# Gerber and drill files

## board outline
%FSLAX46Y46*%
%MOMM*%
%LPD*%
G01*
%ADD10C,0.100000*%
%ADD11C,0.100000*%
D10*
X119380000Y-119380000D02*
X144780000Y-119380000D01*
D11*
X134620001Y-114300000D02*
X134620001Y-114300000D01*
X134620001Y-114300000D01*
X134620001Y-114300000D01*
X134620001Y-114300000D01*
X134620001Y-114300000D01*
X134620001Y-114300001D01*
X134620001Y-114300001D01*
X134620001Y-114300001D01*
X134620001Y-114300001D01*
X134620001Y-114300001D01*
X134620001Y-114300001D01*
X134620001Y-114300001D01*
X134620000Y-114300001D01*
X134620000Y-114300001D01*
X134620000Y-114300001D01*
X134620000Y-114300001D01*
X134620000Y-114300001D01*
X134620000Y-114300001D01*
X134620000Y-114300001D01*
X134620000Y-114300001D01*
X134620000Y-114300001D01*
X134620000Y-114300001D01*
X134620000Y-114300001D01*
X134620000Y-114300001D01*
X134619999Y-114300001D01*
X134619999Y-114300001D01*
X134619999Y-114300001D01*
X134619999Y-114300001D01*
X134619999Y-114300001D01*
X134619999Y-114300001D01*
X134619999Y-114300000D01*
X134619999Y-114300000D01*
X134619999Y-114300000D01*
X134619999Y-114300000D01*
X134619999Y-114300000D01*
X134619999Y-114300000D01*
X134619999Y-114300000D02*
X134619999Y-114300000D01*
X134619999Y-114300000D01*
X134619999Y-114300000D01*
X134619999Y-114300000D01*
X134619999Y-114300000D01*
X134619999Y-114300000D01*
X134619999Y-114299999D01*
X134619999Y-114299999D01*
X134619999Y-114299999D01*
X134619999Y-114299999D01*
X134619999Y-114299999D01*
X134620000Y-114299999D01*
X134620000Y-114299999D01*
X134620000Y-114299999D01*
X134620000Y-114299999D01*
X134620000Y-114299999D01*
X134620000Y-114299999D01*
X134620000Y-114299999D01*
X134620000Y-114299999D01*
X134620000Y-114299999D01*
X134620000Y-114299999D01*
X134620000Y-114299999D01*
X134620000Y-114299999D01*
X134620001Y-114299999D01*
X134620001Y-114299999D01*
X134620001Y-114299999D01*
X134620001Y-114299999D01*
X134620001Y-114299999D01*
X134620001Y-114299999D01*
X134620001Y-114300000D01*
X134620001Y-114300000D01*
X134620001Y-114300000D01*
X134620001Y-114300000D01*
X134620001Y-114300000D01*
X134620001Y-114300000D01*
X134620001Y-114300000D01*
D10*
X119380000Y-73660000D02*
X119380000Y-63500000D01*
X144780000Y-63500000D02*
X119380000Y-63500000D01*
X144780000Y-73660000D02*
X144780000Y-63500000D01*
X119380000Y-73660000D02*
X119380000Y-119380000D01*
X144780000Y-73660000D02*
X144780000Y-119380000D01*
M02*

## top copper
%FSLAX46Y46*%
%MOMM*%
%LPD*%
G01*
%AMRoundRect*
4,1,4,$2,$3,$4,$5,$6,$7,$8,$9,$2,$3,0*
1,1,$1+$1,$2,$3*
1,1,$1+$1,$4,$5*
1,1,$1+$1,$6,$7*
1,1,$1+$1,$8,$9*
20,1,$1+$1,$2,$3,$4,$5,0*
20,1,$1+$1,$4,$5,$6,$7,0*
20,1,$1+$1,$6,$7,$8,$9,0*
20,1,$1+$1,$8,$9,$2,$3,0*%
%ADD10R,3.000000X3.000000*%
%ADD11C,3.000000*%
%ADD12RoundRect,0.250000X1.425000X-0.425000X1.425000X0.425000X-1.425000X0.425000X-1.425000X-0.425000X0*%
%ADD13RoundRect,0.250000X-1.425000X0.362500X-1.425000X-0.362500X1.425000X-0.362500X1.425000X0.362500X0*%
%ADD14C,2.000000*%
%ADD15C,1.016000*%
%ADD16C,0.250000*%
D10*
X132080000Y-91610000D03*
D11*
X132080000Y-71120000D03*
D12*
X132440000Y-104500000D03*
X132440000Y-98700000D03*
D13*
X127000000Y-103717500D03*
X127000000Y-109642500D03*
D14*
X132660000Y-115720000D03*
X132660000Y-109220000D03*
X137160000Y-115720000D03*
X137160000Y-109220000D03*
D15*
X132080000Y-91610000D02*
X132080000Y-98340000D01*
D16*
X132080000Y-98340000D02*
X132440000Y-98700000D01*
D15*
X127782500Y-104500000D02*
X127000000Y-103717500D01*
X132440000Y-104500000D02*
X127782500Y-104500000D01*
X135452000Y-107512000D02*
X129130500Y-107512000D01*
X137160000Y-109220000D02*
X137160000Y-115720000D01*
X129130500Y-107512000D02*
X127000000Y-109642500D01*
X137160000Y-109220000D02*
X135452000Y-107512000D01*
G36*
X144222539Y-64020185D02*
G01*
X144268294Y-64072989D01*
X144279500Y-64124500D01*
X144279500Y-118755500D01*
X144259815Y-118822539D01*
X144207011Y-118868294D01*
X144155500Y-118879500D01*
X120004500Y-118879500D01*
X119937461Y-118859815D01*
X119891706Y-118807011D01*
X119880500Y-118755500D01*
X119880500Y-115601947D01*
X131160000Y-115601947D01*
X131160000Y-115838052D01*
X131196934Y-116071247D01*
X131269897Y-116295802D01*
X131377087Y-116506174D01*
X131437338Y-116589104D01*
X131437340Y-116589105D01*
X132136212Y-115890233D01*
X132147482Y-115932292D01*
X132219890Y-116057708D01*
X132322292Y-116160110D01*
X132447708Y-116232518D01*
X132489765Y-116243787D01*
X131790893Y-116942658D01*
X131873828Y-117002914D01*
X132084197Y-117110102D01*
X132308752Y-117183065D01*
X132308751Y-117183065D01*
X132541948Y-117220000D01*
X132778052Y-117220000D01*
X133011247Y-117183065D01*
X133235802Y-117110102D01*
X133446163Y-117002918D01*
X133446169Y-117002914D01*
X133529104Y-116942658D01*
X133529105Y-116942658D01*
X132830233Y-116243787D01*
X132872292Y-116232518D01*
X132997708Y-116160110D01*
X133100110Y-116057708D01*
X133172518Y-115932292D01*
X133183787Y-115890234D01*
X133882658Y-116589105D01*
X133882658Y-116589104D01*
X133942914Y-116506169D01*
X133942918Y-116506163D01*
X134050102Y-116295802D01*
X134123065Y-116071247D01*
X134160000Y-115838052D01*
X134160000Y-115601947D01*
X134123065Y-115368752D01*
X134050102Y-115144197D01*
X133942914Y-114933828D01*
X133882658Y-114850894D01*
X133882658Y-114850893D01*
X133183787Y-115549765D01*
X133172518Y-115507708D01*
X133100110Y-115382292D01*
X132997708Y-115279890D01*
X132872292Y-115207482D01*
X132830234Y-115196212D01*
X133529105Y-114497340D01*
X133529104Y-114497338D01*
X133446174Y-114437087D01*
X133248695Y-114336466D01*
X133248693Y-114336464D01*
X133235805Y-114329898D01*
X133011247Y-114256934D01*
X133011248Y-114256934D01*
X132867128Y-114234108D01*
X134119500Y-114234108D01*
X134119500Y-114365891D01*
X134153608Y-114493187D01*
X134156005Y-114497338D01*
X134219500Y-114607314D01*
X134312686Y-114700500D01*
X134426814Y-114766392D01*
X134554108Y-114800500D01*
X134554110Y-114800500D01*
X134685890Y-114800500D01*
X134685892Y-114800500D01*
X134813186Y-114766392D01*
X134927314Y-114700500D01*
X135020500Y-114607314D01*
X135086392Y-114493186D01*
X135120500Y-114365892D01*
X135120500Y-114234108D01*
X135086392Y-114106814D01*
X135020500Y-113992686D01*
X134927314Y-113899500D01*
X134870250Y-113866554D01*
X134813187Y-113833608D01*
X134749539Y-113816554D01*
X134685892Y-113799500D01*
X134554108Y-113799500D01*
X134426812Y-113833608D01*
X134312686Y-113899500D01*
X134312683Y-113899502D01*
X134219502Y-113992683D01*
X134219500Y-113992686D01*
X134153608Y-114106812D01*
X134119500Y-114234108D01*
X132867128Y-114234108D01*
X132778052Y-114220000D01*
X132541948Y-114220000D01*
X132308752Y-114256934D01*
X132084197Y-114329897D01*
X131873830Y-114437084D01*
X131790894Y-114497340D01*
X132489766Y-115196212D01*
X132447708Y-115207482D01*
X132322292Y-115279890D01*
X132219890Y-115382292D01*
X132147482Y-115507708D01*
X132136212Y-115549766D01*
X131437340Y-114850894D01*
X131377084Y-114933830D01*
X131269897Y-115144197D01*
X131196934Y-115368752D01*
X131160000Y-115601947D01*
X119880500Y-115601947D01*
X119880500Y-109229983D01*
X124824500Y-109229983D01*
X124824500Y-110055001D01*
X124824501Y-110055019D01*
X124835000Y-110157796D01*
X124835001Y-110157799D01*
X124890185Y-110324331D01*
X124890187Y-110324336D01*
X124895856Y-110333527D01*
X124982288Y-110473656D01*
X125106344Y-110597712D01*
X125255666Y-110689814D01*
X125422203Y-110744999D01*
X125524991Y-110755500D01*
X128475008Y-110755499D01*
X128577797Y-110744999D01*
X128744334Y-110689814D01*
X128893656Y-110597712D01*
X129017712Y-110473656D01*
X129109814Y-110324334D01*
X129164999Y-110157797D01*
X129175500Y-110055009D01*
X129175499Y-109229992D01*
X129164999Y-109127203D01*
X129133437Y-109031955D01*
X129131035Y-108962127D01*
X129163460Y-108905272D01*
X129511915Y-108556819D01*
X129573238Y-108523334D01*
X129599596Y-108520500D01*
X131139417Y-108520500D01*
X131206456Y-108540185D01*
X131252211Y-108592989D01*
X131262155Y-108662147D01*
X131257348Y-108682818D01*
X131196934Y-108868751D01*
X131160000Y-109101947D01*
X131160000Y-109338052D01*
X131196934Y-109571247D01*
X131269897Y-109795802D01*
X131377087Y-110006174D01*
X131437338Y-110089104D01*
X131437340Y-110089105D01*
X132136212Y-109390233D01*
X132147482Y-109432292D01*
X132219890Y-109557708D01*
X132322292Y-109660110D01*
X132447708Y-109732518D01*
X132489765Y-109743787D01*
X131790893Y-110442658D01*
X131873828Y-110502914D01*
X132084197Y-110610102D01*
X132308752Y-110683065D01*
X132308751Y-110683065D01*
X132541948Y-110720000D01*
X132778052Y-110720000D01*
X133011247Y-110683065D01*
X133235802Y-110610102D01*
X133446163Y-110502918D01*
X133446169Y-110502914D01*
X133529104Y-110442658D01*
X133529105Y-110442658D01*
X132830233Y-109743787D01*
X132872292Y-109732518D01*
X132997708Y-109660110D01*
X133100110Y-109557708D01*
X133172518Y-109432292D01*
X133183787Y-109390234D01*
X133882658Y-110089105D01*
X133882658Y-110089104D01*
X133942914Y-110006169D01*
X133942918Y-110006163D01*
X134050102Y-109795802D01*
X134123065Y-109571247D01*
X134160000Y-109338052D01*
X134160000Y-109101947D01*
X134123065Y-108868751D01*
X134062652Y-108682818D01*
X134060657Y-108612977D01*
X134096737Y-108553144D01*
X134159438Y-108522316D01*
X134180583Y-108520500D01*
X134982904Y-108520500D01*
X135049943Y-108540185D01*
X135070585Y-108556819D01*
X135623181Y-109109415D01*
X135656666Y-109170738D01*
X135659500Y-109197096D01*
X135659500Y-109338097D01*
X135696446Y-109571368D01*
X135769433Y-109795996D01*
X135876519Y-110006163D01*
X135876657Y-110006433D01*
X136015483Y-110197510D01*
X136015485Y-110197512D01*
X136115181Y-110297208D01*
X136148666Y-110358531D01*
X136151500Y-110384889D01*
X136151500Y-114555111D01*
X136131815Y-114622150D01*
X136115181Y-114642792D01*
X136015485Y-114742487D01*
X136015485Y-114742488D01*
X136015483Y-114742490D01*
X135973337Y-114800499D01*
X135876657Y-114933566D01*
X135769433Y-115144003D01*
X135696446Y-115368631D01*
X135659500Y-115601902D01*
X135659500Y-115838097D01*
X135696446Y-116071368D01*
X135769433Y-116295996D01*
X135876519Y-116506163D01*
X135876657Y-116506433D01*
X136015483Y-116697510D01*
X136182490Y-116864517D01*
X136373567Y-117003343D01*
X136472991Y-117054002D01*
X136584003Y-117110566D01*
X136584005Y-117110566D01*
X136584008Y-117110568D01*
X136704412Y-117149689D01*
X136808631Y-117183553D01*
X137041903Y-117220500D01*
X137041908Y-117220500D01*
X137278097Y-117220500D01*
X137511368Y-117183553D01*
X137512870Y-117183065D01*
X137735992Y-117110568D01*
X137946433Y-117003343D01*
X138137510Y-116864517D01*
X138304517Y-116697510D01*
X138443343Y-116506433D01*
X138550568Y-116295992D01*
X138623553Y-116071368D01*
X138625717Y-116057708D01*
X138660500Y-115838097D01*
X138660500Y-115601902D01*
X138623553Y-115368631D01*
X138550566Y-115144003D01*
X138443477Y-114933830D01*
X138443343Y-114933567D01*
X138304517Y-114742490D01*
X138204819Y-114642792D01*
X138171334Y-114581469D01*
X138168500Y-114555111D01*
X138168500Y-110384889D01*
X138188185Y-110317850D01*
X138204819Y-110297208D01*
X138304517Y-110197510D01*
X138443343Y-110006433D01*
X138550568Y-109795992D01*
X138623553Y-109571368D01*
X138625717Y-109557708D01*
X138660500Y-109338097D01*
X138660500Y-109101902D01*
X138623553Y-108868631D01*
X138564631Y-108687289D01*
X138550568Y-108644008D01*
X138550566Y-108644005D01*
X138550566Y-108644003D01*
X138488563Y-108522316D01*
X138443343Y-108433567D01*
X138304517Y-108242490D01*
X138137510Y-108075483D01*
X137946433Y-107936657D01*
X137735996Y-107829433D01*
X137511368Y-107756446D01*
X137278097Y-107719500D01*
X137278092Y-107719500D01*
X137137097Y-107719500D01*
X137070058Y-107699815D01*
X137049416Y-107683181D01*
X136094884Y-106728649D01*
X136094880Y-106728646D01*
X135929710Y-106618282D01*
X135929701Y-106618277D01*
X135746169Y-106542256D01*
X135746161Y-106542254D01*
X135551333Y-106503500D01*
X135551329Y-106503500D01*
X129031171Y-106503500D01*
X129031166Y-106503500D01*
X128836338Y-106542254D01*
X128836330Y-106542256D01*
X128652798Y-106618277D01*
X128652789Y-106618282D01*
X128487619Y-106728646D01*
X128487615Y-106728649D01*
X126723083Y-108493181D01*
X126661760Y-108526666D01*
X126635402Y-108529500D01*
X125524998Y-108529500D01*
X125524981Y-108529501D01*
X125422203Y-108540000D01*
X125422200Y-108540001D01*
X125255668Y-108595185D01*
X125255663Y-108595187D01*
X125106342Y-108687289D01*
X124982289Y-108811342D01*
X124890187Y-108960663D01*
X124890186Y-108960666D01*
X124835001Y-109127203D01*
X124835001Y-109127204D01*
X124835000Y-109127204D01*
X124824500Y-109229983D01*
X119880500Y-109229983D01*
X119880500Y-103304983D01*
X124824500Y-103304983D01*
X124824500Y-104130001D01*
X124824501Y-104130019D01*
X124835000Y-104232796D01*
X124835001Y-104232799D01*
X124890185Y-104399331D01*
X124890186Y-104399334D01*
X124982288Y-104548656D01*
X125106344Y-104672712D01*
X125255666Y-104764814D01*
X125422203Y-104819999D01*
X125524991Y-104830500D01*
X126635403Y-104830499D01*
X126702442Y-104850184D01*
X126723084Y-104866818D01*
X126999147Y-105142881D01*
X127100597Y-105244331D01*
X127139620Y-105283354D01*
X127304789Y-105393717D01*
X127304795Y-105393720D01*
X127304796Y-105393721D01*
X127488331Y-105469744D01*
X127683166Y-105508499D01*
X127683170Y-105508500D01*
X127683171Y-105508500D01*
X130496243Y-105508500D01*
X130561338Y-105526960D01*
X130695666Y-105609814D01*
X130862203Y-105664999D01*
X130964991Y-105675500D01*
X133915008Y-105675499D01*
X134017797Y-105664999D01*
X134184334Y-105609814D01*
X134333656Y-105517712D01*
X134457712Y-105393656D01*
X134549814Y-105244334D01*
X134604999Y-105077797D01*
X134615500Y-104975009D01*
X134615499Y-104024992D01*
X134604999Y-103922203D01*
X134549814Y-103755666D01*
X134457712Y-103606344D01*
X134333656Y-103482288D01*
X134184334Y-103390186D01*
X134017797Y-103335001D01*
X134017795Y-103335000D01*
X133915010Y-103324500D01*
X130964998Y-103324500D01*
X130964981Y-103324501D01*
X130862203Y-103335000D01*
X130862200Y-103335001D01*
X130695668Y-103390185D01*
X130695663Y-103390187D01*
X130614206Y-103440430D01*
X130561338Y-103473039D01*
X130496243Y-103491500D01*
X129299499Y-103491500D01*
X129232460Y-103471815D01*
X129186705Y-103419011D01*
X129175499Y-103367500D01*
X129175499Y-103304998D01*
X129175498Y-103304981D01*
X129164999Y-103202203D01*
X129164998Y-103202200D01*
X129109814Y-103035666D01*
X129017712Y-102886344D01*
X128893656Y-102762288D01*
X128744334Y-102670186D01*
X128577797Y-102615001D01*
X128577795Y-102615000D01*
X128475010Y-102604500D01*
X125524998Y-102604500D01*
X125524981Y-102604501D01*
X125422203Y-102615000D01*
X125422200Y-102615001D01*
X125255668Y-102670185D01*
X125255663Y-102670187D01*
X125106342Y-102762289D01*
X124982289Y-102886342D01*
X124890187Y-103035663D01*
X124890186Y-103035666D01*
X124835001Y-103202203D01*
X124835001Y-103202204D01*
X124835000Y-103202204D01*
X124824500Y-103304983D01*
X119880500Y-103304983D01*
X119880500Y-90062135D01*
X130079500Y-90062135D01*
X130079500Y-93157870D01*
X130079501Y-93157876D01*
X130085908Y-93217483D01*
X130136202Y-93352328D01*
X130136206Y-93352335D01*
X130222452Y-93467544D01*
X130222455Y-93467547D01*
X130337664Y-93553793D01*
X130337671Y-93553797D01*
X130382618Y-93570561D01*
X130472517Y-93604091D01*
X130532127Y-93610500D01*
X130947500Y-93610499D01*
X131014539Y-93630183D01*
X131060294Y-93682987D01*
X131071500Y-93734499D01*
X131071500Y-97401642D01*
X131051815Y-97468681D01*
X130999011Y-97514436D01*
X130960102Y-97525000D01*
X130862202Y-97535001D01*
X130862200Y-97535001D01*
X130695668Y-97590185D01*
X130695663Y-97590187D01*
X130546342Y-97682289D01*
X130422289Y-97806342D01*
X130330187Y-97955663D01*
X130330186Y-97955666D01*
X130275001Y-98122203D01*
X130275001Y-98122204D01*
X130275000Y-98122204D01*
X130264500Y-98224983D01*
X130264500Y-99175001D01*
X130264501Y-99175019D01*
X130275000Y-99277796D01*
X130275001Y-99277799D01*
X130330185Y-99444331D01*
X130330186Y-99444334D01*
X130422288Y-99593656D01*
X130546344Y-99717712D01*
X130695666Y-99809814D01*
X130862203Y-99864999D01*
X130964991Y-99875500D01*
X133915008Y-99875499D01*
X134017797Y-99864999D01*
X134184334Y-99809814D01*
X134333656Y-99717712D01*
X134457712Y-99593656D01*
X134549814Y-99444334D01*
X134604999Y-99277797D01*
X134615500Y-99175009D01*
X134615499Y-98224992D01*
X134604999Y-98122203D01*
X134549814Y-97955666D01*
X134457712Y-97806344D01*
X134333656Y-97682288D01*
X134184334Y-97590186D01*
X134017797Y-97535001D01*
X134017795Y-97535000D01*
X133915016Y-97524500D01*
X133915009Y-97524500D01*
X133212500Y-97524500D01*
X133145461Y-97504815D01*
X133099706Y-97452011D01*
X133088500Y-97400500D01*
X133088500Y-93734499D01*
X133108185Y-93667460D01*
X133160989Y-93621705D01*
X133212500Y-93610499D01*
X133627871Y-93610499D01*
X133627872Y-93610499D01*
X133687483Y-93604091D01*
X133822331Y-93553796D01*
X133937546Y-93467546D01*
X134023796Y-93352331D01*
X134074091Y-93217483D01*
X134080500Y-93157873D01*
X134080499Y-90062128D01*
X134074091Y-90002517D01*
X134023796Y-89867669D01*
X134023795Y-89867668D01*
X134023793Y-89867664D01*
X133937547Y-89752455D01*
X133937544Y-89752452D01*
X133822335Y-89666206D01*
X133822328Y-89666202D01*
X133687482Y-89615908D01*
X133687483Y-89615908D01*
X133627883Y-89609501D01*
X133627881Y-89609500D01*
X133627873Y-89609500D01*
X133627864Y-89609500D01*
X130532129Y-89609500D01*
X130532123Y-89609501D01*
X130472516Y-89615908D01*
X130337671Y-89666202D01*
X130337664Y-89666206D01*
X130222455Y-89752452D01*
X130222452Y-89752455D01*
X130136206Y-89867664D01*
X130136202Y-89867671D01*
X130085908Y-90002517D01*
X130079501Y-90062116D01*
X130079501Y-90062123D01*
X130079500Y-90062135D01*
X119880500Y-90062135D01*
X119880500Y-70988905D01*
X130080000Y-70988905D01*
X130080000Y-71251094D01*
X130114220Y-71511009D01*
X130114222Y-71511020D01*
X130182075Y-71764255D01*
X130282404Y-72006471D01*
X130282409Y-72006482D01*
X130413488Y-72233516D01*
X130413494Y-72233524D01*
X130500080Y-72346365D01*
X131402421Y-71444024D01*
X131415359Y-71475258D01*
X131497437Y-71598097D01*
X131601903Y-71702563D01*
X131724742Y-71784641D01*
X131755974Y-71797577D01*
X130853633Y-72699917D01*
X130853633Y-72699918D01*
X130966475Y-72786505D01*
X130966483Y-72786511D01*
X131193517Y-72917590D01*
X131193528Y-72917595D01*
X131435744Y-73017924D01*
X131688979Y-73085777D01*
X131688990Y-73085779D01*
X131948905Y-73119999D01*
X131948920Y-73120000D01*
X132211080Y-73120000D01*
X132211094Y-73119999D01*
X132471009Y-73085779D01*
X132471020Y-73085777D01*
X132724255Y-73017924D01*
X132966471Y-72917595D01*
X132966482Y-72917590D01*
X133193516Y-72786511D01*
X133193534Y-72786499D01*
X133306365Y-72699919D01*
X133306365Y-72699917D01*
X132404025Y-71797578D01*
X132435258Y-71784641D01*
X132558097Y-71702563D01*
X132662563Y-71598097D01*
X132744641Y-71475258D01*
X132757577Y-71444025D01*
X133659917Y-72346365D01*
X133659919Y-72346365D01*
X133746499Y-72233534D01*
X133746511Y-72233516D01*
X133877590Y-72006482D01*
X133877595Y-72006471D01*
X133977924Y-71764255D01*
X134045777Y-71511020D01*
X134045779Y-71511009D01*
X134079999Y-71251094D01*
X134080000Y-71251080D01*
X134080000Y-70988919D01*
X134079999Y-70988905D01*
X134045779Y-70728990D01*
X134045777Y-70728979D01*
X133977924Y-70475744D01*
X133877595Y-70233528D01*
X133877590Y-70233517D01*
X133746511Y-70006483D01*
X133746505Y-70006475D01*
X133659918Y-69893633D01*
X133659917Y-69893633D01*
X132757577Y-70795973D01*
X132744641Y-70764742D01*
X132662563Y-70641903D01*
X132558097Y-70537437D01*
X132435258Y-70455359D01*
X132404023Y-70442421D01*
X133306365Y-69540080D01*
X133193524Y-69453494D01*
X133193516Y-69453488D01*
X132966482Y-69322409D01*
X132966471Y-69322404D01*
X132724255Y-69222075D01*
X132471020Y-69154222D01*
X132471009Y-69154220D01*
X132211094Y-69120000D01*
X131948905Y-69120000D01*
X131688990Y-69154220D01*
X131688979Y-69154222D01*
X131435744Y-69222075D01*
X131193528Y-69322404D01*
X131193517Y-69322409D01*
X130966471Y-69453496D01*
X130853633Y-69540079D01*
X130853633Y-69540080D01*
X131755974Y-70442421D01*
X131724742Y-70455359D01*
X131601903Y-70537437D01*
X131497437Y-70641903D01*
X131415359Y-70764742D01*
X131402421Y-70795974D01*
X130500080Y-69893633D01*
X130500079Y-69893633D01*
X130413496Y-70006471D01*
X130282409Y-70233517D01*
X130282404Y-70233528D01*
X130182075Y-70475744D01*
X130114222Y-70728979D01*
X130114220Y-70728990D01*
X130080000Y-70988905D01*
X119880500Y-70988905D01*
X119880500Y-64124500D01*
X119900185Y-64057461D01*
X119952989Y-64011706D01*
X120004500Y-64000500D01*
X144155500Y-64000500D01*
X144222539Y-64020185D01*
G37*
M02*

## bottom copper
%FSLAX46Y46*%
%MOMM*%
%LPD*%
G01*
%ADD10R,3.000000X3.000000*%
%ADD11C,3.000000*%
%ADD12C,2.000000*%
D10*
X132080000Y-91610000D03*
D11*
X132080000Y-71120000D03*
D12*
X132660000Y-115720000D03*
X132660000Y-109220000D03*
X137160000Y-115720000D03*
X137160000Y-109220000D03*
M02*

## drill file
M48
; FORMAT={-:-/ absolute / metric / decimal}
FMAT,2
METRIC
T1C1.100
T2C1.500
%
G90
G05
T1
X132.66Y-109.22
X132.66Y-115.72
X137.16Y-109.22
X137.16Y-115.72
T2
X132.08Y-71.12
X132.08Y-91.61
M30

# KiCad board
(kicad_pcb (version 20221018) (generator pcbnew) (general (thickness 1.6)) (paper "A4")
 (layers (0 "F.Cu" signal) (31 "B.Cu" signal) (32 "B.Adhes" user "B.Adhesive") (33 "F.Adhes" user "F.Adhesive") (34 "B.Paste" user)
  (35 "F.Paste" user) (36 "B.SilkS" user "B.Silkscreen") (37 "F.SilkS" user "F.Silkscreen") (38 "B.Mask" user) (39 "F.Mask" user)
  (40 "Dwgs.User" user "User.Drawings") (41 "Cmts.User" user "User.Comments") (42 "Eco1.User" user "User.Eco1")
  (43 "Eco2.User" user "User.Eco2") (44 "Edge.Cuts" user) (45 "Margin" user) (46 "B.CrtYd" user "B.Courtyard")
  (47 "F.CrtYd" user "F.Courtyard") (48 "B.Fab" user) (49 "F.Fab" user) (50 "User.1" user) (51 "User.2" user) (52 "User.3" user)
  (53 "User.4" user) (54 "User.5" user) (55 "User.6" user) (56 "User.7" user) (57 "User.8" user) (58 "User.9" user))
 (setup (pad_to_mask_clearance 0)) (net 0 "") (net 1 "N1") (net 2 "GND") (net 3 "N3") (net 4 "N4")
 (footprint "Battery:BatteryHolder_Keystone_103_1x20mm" (layer "F.Cu") (at 132.08 91.61 90)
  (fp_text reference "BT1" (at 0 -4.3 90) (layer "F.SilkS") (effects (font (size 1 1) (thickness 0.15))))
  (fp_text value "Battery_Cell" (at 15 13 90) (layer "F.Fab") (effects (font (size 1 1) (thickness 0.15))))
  (pad "1" thru_hole rect (at 0 0 90) (size 3 3) (drill 1.5) (layers "*.Cu" "*.Mask") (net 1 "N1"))
  (pad "2" thru_hole circle (at 20.49 0 90) (size 3 3) (drill 1.5) (layers "*.Cu" "*.Mask") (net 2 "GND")))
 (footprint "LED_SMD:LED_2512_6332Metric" (layer "F.Cu") (at 132.44 101.6 90)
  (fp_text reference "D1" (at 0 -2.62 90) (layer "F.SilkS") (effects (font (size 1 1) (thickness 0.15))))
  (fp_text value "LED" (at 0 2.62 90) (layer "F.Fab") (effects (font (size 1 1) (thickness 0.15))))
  (pad "1" smd roundrect (at -2.9 0 90) (size 1.35 3.35) (layers "F.Cu" "F.Paste" "F.Mask") (roundrect_rratio 0.185185) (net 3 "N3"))
  (pad "2" smd roundrect (at 2.9 0 90) (size 1.35 3.35) (layers "F.Cu" "F.Paste" "F.Mask") (roundrect_rratio 0.185185) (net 1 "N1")))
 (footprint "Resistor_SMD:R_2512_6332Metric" (layer "F.Cu") (at 127 106.68 -90)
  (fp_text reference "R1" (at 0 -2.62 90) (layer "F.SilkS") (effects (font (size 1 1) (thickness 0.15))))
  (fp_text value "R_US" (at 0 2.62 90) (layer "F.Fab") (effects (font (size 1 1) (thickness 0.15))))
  (pad "1" smd roundrect (at -2.9625 0 270) (size 1.225 3.35) (layers "F.Cu" "F.Paste" "F.Mask") (roundrect_rratio 0.204082) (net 3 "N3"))
  (pad "2" smd roundrect (at 2.9625 0 270) (size 1.225 3.35) (layers "F.Cu" "F.Paste" "F.Mask") (roundrect_rratio 0.204082) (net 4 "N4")))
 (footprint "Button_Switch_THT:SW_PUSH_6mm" (layer "F.Cu") (at 132.66 115.72 90)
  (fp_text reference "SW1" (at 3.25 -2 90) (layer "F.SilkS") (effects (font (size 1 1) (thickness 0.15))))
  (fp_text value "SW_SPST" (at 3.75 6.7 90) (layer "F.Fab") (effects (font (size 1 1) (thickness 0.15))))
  (pad "1" thru_hole circle (at 0 0 180) (size 2 2) (drill 1.1) (layers "*.Cu" "*.Mask") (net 2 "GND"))
  (pad "1" thru_hole circle (at 6.5 0 180) (size 2 2) (drill 1.1) (layers "*.Cu" "*.Mask") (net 2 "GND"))
  (pad "2" thru_hole circle (at 0 4.5 180) (size 2 2) (drill 1.1) (layers "*.Cu" "*.Mask") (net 4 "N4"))
  (pad "2" thru_hole circle (at 6.5 4.5 180) (size 2 2) (drill 1.1) (layers "*.Cu" "*.Mask") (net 4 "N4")))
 (gr_line (start 119.38 119.38) (end 144.78 119.38) (stroke (width 0.1) (type default)) (layer "Edge.Cuts"))
 (gr_arc (start 134.62 114.3) (mid 134.62 114.3) (end 134.62 114.3) (stroke (width 0.1) (type default)) (layer "Edge.Cuts"))
 (gr_line (start 119.38 73.66) (end 119.38 63.5) (stroke (width 0.1) (type default)) (layer "Edge.Cuts"))
 (gr_line (start 144.78 63.5) (end 119.38 63.5) (stroke (width 0.1) (type default)) (layer "Edge.Cuts"))
 (gr_line (start 144.78 73.66) (end 144.78 63.5) (stroke (width 0.1) (type default)) (layer "Edge.Cuts"))
 (gr_line (start 119.38 73.66) (end 119.38 119.38) (stroke (width 0.1) (type default)) (layer "Edge.Cuts"))
 (gr_line (start 144.78 73.66) (end 144.78 119.38) (stroke (width 0.1) (type default)) (layer "Edge.Cuts"))
 (segment (start 132.08 91.61) (end 132.08 98.34) (width 1.016) (layer "F.Cu") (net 1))
 (segment (start 132.08 98.34) (end 132.44 98.7) (width 0.25) (layer "F.Cu") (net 1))
 (segment (start 127.7825 104.5) (end 127 103.7175) (width 1.016) (layer "F.Cu") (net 3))
 (segment (start 132.44 104.5) (end 127.7825 104.5) (width 1.016) (layer "F.Cu") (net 3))
 (segment (start 135.452 107.512) (end 129.1305 107.512) (width 1.016) (layer "F.Cu") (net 4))
 (segment (start 137.16 109.22) (end 137.16 115.72) (width 1.016) (layer "F.Cu") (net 4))
 (segment (start 129.1305 107.512) (end 127 109.6425) (width 1.016) (layer "F.Cu") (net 4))
 (segment (start 137.16 109.22) (end 135.452 107.512) (width 1.016) (layer "F.Cu") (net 4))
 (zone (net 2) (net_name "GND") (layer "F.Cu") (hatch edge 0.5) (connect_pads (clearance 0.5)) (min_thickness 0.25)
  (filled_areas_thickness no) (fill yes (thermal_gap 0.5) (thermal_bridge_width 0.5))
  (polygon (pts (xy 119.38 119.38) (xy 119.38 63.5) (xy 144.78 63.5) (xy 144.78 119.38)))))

